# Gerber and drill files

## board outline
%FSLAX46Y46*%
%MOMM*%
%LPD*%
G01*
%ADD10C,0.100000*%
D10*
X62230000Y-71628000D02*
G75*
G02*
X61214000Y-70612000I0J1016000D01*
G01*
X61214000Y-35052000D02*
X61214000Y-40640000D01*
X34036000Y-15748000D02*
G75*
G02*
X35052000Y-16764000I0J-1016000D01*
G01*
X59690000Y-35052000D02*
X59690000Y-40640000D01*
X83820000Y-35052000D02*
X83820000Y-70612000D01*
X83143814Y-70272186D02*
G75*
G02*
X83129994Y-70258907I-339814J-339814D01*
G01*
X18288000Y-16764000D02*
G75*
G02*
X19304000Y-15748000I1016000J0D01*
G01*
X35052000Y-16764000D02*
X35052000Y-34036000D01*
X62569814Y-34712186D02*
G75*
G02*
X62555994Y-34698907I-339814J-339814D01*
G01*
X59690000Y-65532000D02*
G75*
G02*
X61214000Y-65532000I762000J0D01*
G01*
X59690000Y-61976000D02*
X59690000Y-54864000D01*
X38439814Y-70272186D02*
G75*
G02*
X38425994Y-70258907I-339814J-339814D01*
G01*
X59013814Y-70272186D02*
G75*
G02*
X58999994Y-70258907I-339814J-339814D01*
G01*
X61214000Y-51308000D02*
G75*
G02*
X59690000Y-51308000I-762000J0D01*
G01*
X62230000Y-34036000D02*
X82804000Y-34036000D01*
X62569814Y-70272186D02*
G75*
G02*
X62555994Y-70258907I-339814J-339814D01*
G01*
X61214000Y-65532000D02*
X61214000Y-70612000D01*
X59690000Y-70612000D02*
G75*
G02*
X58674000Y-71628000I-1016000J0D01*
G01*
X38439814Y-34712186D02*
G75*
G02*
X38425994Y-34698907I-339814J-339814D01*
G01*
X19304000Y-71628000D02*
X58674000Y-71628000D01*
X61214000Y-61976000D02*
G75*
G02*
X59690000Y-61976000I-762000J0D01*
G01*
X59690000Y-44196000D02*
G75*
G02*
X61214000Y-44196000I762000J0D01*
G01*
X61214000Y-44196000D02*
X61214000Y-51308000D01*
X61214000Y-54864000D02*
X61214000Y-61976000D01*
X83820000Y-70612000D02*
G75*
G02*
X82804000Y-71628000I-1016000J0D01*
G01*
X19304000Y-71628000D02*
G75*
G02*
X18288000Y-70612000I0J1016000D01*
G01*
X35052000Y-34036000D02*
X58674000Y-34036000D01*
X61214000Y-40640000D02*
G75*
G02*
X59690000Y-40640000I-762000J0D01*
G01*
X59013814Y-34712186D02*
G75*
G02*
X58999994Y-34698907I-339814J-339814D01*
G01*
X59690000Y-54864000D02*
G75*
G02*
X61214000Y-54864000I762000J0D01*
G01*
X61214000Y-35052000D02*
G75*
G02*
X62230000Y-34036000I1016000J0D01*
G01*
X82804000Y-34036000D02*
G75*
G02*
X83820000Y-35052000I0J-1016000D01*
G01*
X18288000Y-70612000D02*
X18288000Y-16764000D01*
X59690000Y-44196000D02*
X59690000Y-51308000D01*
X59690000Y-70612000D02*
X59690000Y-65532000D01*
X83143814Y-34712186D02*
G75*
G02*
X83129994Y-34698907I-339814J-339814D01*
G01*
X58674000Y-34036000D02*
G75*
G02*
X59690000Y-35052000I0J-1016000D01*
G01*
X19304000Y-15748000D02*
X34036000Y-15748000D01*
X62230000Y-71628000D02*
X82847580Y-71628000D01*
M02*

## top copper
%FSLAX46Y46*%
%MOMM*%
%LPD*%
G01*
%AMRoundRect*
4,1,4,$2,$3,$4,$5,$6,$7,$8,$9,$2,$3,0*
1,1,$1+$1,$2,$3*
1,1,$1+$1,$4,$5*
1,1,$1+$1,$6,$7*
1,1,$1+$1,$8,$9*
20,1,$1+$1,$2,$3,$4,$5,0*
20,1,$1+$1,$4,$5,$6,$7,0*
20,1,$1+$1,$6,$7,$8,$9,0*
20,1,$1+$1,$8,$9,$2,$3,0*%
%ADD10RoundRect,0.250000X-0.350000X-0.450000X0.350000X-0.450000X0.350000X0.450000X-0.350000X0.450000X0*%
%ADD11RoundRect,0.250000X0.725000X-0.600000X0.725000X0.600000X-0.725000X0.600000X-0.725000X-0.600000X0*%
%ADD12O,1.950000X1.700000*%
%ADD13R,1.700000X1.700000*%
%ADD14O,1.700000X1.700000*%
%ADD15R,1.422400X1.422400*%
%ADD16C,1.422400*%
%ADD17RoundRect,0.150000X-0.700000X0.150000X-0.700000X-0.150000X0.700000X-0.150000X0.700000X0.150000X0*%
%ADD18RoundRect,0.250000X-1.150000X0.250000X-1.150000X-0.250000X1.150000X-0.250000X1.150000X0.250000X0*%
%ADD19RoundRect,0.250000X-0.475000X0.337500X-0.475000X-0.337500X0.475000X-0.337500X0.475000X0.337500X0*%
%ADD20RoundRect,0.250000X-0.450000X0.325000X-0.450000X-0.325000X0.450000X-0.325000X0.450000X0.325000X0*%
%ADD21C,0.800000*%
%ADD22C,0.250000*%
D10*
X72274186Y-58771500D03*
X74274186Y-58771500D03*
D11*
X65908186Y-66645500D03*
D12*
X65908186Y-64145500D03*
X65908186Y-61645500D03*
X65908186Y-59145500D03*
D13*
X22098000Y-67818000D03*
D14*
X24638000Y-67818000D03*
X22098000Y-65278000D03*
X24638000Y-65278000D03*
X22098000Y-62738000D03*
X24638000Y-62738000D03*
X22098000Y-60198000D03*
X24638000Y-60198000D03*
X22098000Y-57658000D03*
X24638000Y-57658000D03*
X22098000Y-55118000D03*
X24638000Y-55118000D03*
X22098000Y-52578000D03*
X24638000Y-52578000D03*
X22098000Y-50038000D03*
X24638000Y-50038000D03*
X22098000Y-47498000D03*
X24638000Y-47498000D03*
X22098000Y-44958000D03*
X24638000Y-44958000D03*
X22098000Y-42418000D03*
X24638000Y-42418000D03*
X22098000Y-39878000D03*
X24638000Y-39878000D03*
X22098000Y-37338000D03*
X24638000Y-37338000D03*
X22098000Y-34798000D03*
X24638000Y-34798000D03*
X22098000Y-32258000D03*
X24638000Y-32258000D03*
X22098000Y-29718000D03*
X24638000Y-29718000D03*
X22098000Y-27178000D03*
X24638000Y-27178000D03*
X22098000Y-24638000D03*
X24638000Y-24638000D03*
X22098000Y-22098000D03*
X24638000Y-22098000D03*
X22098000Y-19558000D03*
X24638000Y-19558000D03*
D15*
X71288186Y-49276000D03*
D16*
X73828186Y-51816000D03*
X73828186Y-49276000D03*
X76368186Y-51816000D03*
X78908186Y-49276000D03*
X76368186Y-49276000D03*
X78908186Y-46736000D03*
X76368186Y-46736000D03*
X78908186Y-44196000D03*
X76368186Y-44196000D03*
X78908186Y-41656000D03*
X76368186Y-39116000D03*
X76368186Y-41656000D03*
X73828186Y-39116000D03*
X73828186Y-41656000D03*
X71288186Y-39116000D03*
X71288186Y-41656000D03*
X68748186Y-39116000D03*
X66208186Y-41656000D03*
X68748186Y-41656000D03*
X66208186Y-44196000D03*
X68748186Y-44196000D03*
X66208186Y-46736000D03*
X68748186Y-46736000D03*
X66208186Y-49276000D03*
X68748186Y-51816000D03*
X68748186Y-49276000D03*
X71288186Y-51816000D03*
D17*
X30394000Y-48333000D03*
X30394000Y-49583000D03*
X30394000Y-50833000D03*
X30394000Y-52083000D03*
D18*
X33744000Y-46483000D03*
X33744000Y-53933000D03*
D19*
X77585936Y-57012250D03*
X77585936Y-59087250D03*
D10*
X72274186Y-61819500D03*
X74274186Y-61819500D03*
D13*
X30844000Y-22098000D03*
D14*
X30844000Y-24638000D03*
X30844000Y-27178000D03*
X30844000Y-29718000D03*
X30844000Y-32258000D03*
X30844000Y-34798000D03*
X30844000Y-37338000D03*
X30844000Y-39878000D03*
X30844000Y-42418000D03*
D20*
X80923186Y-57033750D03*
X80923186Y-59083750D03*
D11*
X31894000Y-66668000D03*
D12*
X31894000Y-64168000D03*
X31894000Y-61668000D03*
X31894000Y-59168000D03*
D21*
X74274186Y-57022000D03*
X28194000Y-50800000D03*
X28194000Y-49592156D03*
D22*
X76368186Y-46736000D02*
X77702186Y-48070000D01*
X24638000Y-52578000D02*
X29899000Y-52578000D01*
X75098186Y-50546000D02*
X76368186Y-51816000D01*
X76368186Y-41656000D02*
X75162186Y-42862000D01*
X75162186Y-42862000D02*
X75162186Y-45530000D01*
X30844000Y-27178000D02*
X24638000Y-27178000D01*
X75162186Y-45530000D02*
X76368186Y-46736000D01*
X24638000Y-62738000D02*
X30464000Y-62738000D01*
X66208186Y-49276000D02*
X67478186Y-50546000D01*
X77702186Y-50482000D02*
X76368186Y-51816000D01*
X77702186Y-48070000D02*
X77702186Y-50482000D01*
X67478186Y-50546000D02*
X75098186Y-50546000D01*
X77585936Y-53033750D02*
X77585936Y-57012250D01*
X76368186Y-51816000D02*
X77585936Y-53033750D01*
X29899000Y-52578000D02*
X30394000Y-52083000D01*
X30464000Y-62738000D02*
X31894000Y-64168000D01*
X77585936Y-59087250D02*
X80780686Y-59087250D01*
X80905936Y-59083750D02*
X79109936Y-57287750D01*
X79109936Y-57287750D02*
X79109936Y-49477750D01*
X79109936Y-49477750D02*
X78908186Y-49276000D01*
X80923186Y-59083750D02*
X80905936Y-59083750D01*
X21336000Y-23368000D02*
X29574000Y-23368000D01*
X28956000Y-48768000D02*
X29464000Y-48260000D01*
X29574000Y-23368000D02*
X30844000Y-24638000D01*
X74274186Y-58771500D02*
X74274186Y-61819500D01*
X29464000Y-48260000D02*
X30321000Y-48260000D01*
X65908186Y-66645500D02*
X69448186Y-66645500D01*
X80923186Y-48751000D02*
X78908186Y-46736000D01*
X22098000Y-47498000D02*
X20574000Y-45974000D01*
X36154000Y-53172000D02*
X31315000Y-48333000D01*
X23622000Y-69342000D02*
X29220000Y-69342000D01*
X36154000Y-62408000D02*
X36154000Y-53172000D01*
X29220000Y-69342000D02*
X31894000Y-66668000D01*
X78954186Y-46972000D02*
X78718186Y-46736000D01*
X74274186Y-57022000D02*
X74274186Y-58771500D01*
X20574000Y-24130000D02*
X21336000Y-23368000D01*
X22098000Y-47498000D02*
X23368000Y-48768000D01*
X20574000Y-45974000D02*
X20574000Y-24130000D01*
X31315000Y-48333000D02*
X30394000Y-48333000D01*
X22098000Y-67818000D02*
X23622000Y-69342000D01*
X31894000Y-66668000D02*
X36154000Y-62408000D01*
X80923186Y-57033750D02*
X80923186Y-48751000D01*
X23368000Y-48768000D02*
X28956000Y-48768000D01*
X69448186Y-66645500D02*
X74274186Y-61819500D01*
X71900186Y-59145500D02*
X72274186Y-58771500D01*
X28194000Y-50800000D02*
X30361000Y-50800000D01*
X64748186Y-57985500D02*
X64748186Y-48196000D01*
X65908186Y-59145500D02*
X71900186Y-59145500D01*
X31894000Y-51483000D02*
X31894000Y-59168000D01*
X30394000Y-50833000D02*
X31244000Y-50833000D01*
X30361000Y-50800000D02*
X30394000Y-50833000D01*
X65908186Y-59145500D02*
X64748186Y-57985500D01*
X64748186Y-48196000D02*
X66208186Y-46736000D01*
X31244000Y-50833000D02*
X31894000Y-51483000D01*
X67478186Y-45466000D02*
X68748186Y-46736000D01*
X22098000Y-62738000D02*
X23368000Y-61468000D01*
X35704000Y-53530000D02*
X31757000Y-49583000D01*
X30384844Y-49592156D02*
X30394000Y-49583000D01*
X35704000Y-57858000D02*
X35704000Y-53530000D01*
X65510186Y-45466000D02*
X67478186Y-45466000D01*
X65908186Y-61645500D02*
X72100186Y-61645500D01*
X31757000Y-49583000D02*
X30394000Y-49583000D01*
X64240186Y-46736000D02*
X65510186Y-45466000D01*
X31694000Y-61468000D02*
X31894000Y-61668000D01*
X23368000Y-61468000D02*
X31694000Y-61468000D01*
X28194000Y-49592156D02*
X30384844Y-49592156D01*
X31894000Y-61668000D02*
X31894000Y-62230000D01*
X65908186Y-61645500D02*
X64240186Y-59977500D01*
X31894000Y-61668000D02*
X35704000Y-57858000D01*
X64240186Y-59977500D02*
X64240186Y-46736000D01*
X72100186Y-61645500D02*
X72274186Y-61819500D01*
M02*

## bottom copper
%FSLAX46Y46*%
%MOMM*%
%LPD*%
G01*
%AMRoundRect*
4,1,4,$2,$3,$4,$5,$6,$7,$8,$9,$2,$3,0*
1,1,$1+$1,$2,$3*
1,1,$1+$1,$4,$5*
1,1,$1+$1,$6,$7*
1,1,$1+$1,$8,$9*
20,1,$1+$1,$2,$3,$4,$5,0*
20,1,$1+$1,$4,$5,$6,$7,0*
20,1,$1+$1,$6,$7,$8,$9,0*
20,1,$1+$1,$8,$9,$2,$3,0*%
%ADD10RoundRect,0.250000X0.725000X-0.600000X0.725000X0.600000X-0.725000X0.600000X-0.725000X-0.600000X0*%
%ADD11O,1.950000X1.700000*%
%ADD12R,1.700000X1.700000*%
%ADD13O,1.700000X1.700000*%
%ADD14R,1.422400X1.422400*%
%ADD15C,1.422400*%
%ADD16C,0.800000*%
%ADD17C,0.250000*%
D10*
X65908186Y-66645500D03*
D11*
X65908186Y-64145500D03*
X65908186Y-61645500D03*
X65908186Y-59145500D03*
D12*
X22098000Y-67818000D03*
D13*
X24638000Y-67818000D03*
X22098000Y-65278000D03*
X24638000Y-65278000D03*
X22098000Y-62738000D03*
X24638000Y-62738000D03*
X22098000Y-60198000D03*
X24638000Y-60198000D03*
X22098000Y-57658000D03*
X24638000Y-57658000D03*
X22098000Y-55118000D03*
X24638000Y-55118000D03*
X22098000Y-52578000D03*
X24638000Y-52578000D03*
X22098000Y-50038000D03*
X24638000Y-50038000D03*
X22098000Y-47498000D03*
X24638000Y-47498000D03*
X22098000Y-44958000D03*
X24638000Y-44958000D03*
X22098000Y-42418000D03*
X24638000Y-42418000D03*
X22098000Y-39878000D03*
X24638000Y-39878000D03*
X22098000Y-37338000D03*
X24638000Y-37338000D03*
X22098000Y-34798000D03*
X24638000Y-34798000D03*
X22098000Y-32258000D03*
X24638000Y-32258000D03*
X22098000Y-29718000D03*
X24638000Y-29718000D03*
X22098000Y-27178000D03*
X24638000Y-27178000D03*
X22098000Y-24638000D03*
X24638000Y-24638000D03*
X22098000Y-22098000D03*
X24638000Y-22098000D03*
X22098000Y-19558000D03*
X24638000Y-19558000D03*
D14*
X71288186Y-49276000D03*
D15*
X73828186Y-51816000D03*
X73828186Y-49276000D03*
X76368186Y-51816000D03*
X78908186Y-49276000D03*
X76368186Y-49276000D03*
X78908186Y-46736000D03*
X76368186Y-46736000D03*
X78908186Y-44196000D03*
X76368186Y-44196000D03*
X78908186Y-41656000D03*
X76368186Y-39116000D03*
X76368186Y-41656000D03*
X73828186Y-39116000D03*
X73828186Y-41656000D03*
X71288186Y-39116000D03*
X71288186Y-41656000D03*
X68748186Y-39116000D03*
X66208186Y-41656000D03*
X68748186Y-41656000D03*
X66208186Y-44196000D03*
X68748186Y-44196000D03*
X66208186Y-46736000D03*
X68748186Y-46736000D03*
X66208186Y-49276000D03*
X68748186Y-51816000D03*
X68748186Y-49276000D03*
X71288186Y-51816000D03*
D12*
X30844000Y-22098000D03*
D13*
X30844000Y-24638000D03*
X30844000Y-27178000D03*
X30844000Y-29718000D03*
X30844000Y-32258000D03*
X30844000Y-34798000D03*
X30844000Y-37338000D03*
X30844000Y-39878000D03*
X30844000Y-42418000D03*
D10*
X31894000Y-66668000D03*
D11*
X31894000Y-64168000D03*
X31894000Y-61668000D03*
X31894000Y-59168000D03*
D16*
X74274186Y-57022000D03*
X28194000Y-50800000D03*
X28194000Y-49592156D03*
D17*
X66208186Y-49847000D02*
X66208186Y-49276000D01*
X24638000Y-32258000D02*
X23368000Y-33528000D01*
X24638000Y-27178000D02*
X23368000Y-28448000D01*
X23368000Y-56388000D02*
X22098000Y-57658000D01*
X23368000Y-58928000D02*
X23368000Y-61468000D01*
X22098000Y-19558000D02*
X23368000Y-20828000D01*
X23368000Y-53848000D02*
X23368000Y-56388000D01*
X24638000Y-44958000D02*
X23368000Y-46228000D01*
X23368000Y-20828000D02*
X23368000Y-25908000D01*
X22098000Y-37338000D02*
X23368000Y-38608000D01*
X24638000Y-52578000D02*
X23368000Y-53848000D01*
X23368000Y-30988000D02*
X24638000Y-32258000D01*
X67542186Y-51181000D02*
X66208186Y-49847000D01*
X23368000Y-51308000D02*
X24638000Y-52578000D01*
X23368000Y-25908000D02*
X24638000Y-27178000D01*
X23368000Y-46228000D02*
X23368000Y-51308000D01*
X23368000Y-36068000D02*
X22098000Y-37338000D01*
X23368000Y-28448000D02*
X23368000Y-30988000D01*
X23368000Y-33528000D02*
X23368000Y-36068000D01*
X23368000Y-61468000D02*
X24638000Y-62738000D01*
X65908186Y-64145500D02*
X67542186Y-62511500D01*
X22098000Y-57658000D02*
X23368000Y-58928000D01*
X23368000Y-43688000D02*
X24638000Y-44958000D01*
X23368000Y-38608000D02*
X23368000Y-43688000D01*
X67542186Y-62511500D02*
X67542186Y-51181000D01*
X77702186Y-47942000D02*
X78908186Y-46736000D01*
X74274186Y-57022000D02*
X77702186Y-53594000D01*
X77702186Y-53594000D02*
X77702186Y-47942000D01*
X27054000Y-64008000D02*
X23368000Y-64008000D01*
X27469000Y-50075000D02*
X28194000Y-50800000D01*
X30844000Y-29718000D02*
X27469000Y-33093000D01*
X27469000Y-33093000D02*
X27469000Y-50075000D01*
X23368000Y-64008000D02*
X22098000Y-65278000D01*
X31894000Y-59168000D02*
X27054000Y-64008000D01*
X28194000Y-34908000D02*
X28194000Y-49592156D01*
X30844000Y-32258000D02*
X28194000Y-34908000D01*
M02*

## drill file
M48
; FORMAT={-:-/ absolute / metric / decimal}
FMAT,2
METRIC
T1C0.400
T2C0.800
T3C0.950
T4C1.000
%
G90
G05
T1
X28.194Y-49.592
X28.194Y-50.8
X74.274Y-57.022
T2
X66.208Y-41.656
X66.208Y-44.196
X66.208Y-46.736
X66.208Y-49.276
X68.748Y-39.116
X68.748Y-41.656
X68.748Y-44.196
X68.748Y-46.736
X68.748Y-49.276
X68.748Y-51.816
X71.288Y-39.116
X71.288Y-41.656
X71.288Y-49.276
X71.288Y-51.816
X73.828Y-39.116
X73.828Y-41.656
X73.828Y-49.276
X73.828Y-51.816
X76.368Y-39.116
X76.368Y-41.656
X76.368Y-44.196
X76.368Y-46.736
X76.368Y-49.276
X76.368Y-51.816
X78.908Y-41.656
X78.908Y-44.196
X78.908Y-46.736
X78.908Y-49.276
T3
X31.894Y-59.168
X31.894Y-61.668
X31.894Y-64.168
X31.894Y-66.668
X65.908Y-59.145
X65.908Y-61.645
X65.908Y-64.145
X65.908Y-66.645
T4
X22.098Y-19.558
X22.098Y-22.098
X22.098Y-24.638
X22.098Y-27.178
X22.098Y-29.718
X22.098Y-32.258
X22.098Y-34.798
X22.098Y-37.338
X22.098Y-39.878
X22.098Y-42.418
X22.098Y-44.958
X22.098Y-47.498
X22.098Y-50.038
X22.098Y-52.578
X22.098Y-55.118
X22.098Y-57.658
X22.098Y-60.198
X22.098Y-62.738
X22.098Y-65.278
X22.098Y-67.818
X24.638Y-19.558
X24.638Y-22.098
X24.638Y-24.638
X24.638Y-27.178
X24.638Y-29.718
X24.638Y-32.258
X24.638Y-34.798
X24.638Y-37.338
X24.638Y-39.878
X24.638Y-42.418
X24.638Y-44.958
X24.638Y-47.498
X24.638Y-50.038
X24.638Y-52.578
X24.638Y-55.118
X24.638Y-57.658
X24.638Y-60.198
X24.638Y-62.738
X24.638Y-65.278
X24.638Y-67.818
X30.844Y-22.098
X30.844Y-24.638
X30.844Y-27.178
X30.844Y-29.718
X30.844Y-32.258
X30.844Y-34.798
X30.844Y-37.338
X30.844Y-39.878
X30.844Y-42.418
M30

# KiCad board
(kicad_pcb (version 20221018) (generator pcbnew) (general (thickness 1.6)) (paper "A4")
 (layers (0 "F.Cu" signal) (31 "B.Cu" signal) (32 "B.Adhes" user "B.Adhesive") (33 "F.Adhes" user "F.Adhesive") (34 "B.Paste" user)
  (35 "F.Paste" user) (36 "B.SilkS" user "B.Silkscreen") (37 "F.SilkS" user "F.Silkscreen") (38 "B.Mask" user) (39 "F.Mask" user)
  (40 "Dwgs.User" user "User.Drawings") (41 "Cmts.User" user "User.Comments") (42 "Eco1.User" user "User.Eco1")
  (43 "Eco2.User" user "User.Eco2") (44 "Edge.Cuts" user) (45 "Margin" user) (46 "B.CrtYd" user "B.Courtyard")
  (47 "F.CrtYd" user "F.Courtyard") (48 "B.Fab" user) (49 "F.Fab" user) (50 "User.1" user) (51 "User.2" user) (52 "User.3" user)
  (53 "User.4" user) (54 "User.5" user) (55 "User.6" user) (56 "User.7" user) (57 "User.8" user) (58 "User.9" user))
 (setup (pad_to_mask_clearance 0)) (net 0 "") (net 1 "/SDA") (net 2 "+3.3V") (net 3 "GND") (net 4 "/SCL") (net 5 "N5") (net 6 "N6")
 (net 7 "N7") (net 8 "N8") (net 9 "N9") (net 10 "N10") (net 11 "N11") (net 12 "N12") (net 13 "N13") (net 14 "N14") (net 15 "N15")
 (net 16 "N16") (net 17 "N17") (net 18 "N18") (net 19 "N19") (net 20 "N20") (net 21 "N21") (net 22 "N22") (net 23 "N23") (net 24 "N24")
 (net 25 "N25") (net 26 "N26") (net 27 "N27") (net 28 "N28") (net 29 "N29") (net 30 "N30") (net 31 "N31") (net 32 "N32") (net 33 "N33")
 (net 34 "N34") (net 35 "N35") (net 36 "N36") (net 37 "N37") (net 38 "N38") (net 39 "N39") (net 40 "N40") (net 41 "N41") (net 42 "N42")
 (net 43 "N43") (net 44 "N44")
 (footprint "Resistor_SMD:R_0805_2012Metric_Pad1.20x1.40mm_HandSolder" (layer "F.Cu") (at 73.274186 58.7715)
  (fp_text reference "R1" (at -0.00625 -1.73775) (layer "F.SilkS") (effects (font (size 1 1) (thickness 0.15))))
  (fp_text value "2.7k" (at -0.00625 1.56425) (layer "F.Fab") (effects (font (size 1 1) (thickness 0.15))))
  (pad "1" smd roundrect (at -1 0) (size 1.2 1.4) (layers "F.Cu" "F.Paste" "F.Mask") (roundrect_rratio 0.208333) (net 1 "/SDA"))
  (pad "2" smd roundrect (at 1 0) (size 1.2 1.4) (layers "F.Cu" "F.Paste" "F.Mask") (roundrect_rratio 0.208333) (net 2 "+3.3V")))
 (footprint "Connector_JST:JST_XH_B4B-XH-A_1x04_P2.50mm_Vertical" (layer "F.Cu") (at 65.908186 66.6455 90)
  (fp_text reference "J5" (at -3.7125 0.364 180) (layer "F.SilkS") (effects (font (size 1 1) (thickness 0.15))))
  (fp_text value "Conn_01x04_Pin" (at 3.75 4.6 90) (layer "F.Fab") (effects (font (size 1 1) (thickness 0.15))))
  (pad "1" thru_hole roundrect (at 0 0 90) (size 1.7 1.95) (drill 0.95) (layers "*.Cu" "*.Mask") (roundrect_rratio 0.147059) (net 2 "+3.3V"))
  (pad "2" thru_hole oval (at 2.5 0 90) (size 1.7 1.95) (drill 0.95) (layers "*.Cu" "*.Mask") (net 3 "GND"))
  (pad "3" thru_hole oval (at 5 0 90) (size 1.7 1.95) (drill 0.95) (layers "*.Cu" "*.Mask") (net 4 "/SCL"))
  (pad "4" thru_hole oval (at 7.5 0 90) (size 1.7 1.95) (drill 0.95) (layers "*.Cu" "*.Mask") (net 1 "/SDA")))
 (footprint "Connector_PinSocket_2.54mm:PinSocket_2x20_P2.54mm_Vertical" (layer "F.Cu") (at 22.098 67.818 180)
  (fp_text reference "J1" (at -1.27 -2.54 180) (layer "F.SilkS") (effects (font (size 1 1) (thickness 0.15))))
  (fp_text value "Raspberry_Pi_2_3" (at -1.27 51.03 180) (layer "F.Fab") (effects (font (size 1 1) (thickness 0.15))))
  (pad "1" thru_hole rect (at 0 0 180) (size 1.7 1.7) (drill 1) (layers "*.Cu" "*.Mask") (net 2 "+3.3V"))
  (pad "2" thru_hole oval (at -2.54 0 180) (size 1.7 1.7) (drill 1) (layers "*.Cu" "*.Mask") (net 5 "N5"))
  (pad "3" thru_hole oval (at 0 2.54 180) (size 1.7 1.7) (drill 1) (layers "*.Cu" "*.Mask") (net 1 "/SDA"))
  (pad "4" thru_hole oval (at -2.54 2.54 180) (size 1.7 1.7) (drill 1) (layers "*.Cu" "*.Mask") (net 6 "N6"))
  (pad "5" thru_hole oval (at 0 5.08 180) (size 1.7 1.7) (drill 1) (layers "*.Cu" "*.Mask") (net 4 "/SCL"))
  (pad "6" thru_hole oval (at -2.54 5.08 180) (size 1.7 1.7) (drill 1) (layers "*.Cu" "*.Mask") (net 3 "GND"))
  (pad "7" thru_hole oval (at 0 7.62 180) (size 1.7 1.7) (drill 1) (layers "*.Cu" "*.Mask") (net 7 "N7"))
  (pad "8" thru_hole oval (at -2.54 7.62 180) (size 1.7 1.7) (drill 1) (layers "*.Cu" "*.Mask") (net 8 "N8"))
  (pad "9" thru_hole oval (at 0 10.16 180) (size 1.7 1.7) (drill 1) (layers "*.Cu" "*.Mask") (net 3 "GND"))
  (pad "10" thru_hole oval (at -2.54 10.16 180) (size 1.7 1.7) (drill 1) (layers "*.Cu" "*.Mask") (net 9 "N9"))
  (pad "11" thru_hole oval (at 0 12.7 180) (size 1.7 1.7) (drill 1) (layers "*.Cu" "*.Mask") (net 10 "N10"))
  (pad "12" thru_hole oval (at -2.54 12.7 180) (size 1.7 1.7) (drill 1) (layers "*.Cu" "*.Mask") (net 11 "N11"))
  (pad "13" thru_hole oval (at 0 15.24 180) (size 1.7 1.7) (drill 1) (layers "*.Cu" "*.Mask") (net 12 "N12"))
  (pad "14" thru_hole oval (at -2.54 15.24 180) (size 1.7 1.7) (drill 1) (layers "*.Cu" "*.Mask") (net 3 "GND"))
  (pad "15" thru_hole oval (at 0 17.78 180) (size 1.7 1.7) (drill 1) (layers "*.Cu" "*.Mask") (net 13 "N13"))
  (pad "16" thru_hole oval (at -2.54 17.78 180) (size 1.7 1.7) (drill 1) (layers "*.Cu" "*.Mask") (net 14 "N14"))
  (pad "17" thru_hole oval (at 0 20.32 180) (size 1.7 1.7) (drill 1) (layers "*.Cu" "*.Mask") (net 2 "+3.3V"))
  (pad "18" thru_hole oval (at -2.54 20.32 180) (size 1.7 1.7) (drill 1) (layers "*.Cu" "*.Mask") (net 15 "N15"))
  (pad "19" thru_hole oval (at 0 22.86 180) (size 1.7 1.7) (drill 1) (layers "*.Cu" "*.Mask") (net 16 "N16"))
  (pad "20" thru_hole oval (at -2.54 22.86 180) (size 1.7 1.7) (drill 1) (layers "*.Cu" "*.Mask") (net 3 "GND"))
  (pad "21" thru_hole oval (at 0 25.4 180) (size 1.7 1.7) (drill 1) (layers "*.Cu" "*.Mask") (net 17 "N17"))
  (pad "22" thru_hole oval (at -2.54 25.4 180) (size 1.7 1.7) (drill 1) (layers "*.Cu" "*.Mask") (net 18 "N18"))
  (pad "23" thru_hole oval (at 0 27.94 180) (size 1.7 1.7) (drill 1) (layers "*.Cu" "*.Mask") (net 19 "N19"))
  (pad "24" thru_hole oval (at -2.54 27.94 180) (size 1.7 1.7) (drill 1) (layers "*.Cu" "*.Mask") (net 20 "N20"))
  (pad "25" thru_hole oval (at 0 30.48 180) (size 1.7 1.7) (drill 1) (layers "*.Cu" "*.Mask") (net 3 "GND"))
  (pad "26" thru_hole oval (at -2.54 30.48 180) (size 1.7 1.7) (drill 1) (layers "*.Cu" "*.Mask") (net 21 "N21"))
  (pad "27" thru_hole oval (at 0 33.02 180) (size 1.7 1.7) (drill 1) (layers "*.Cu" "*.Mask") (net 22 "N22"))
  (pad "28" thru_hole oval (at -2.54 33.02 180) (size 1.7 1.7) (drill 1) (layers "*.Cu" "*.Mask") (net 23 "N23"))
  (pad "29" thru_hole oval (at 0 35.56 180) (size 1.7 1.7) (drill 1) (layers "*.Cu" "*.Mask") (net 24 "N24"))
  (pad "30" thru_hole oval (at -2.54 35.56 180) (size 1.7 1.7) (drill 1) (layers "*.Cu" "*.Mask") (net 3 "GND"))
  (pad "31" thru_hole oval (at 0 38.1 180) (size 1.7 1.7) (drill 1) (layers "*.Cu" "*.Mask") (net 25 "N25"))
  (pad "32" thru_hole oval (at -2.54 38.1 180) (size 1.7 1.7) (drill 1) (layers "*.Cu" "*.Mask") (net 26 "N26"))
  (pad "33" thru_hole oval (at 0 40.64 180) (size 1.7 1.7) (drill 1) (layers "*.Cu" "*.Mask") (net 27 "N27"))
  (pad "34" thru_hole oval (at -2.54 40.64 180) (size 1.7 1.7) (drill 1) (layers "*.Cu" "*.Mask") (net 3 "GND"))
  (pad "35" thru_hole oval (at 0 43.18 180) (size 1.7 1.7) (drill 1) (layers "*.Cu" "*.Mask") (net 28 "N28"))
  (pad "36" thru_hole oval (at -2.54 43.18 180) (size 1.7 1.7) (drill 1) (layers "*.Cu" "*.Mask") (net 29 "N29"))
  (pad "37" thru_hole oval (at 0 45.72 180) (size 1.7 1.7) (drill 1) (layers "*.Cu" "*.Mask") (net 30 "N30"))
  (pad "38" thru_hole oval (at -2.54 45.72 180) (size 1.7 1.7) (drill 1) (layers "*.Cu" "*.Mask") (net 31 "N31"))
  (pad "39" thru_hole oval (at 0 48.26 180) (size 1.7 1.7) (drill 1) (layers "*.Cu" "*.Mask") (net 3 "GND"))
  (pad "40" thru_hole oval (at -2.54 48.26 180) (size 1.7 1.7) (drill 1) (layers "*.Cu" "*.Mask") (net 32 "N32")))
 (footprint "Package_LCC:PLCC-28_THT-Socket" (layer "F.Cu") (at 71.288186 49.276 180)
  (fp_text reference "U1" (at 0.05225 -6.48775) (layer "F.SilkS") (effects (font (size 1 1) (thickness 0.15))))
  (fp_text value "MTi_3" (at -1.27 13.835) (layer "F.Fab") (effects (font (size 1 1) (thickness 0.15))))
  (pad "1" thru_hole rect (at 0 0 180) (size 1.4224 1.4224) (drill 0.8) (layers "*.Cu" "*.Mask"))
  (pad "2" thru_hole circle (at -2.54 -2.54 180) (size 1.4224 1.4224) (drill 0.8) (layers "*.Cu" "*.Mask"))
  (pad "3" thru_hole circle (at -2.54 0 180) (size 1.4224 1.4224) (drill 0.8) (layers "*.Cu" "*.Mask"))
  (pad "4" thru_hole circle (at -5.08 -2.54 180) (size 1.4224 1.4224) (drill 0.8) (layers "*.Cu" "*.Mask") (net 3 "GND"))
  (pad "5" thru_hole circle (at -7.62 0 180) (size 1.4224 1.4224) (drill 0.8) (layers "*.Cu" "*.Mask") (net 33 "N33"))
  (pad "6" thru_hole circle (at -5.08 0 180) (size 1.4224 1.4224) (drill 0.8) (layers "*.Cu" "*.Mask") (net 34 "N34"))
  (pad "7" thru_hole circle (at -7.62 2.54 180) (size 1.4224 1.4224) (drill 0.8) (layers "*.Cu" "*.Mask") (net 2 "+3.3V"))
  (pad "8" thru_hole circle (at -5.08 2.54 180) (size 1.4224 1.4224) (drill 0.8) (layers "*.Cu" "*.Mask") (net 3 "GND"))
  (pad "9" thru_hole circle (at -7.62 5.08 180) (size 1.4224 1.4224) (drill 0.8) (layers "*.Cu" "*.Mask"))
  (pad "10" thru_hole circle (at -5.08 5.08 180) (size 1.4224 1.4224) (drill 0.8) (layers "*.Cu" "*.Mask") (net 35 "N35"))
  (pad "11" thru_hole circle (at -7.62 7.62 180) (size 1.4224 1.4224) (drill 0.8) (layers "*.Cu" "*.Mask") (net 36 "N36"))
  (pad "12" thru_hole circle (at -5.08 10.16 180) (size 1.4224 1.4224) (drill 0.8) (layers "*.Cu" "*.Mask") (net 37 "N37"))
  (pad "13" thru_hole circle (at -5.08 7.62 180) (size 1.4224 1.4224) (drill 0.8) (layers "*.Cu" "*.Mask") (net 3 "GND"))
  (pad "14" thru_hole circle (at -2.54 10.16 180) (size 1.4224 1.4224) (drill 0.8) (layers "*.Cu" "*.Mask") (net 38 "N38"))
  (pad "15" thru_hole circle (at -2.54 7.62 180) (size 1.4224 1.4224) (drill 0.8) (layers "*.Cu" "*.Mask") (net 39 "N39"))
  (pad "16" thru_hole circle (at 0 10.16 180) (size 1.4224 1.4224) (drill 0.8) (layers "*.Cu" "*.Mask"))
  (pad "17" thru_hole circle (at 0 7.62 180) (size 1.4224 1.4224) (drill 0.8) (layers "*.Cu" "*.Mask"))
  (pad "18" thru_hole circle (at 2.54 10.16 180) (size 1.4224 1.4224) (drill 0.8) (layers "*.Cu" "*.Mask"))
  (pad "19" thru_hole circle (at 5.08 7.62 180) (size 1.4224 1.4224) (drill 0.8) (layers "*.Cu" "*.Mask"))
  (pad "20" thru_hole circle (at 2.54 7.62 180) (size 1.4224 1.4224) (drill 0.8) (layers "*.Cu" "*.Mask"))
  (pad "21" thru_hole circle (at 5.08 5.08 180) (size 1.4224 1.4224) (drill 0.8) (layers "*.Cu" "*.Mask"))
  (pad "22" thru_hole circle (at 2.54 5.08 180) (size 1.4224 1.4224) (drill 0.8) (layers "*.Cu" "*.Mask"))
  (pad "23" thru_hole circle (at 5.08 2.54 180) (size 1.4224 1.4224) (drill 0.8) (layers "*.Cu" "*.Mask") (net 1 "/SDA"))
  (pad "24" thru_hole circle (at 2.54 2.54 180) (size 1.4224 1.4224) (drill 0.8) (layers "*.Cu" "*.Mask") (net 4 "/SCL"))
  (pad "25" thru_hole circle (at 5.08 0 180) (size 1.4224 1.4224) (drill 0.8) (layers "*.Cu" "*.Mask") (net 3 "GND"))
  (pad "26" thru_hole circle (at 2.54 -2.54 180) (size 1.4224 1.4224) (drill 0.8) (layers "*.Cu" "*.Mask"))
  (pad "27" thru_hole circle (at 2.54 0 180) (size 1.4224 1.4224) (drill 0.8) (layers "*.Cu" "*.Mask"))
  (pad "28" thru_hole circle (at 0 -2.54 180) (size 1.4224 1.4224) (drill 0.8) (layers "*.Cu" "*.Mask")))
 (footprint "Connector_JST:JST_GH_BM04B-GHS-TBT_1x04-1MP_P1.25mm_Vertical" (layer "F.Cu") (at 32.344 50.208 -90)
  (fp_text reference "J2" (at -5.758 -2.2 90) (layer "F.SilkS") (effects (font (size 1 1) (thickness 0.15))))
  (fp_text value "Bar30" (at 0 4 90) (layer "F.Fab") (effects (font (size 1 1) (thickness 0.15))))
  (pad "1" smd roundrect (at -1.875 1.95 270) (size 0.6 1.7) (layers "F.Cu" "F.Paste" "F.Mask") (roundrect_rratio 0.25) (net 2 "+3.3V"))
  (pad "2" smd roundrect (at -0.625 1.95 270) (size 0.6 1.7) (layers "F.Cu" "F.Paste" "F.Mask") (roundrect_rratio 0.25) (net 4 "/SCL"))
  (pad "3" smd roundrect (at 0.625 1.95 270) (size 0.6 1.7) (layers "F.Cu" "F.Paste" "F.Mask") (roundrect_rratio 0.25) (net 1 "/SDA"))
  (pad "4" smd roundrect (at 1.875 1.95 270) (size 0.6 1.7) (layers "F.Cu" "F.Paste" "F.Mask") (roundrect_rratio 0.25) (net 3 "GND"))
  (pad "MP" smd roundrect (at -3.725 -1.4 270) (size 1 2.8) (layers "F.Cu" "F.Paste" "F.Mask") (roundrect_rratio 0.25))
  (pad "MP" smd roundrect (at 3.725 -1.4 270) (size 1 2.8) (layers "F.Cu" "F.Paste" "F.Mask") (roundrect_rratio 0.25)))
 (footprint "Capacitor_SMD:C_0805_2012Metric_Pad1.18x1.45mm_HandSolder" (layer "F.Cu") (at 77.585936 58.04975 -90)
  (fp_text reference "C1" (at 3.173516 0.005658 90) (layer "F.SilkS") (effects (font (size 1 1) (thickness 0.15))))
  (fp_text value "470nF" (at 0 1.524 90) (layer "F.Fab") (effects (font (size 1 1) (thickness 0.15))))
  (pad "1" smd roundrect (at -1.0375 0 270) (size 1.175 1.45) (layers "F.Cu" "F.Paste" "F.Mask") (roundrect_rratio 0.212766) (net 3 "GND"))
  (pad "2" smd roundrect (at 1.0375 0 270) (size 1.175 1.45) (layers "F.Cu" "F.Paste" "F.Mask") (roundrect_rratio 0.212766) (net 33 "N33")))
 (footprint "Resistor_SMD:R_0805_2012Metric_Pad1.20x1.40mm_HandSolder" (layer "F.Cu") (at 73.274186 61.8195)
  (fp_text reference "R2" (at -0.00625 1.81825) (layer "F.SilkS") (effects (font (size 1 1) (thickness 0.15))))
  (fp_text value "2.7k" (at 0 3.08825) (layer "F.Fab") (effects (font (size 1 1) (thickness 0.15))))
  (pad "1" smd roundrect (at -1 0) (size 1.2 1.4) (layers "F.Cu" "F.Paste" "F.Mask") (roundrect_rratio 0.208333) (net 4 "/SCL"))
  (pad "2" smd roundrect (at 1 0) (size 1.2 1.4) (layers "F.Cu" "F.Paste" "F.Mask") (roundrect_rratio 0.208333) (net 2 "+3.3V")))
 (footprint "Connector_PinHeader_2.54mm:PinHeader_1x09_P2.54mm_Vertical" (layer "F.Cu") (at 30.844 22.098)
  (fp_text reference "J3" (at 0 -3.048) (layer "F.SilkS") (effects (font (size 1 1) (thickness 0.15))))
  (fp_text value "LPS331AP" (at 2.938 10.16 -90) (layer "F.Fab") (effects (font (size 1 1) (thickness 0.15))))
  (pad "1" thru_hole rect (at 0 0) (size 1.7 1.7) (drill 1) (layers "*.Cu" "*.Mask") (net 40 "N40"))
  (pad "2" thru_hole oval (at 0 2.54) (size 1.7 1.7) (drill 1) (layers "*.Cu" "*.Mask") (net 2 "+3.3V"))
  (pad "3" thru_hole oval (at 0 5.08) (size 1.7 1.7) (drill 1) (layers "*.Cu" "*.Mask") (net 3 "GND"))
  (pad "4" thru_hole oval (at 0 7.62) (size 1.7 1.7) (drill 1) (layers "*.Cu" "*.Mask") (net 1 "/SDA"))
  (pad "5" thru_hole oval (at 0 10.16) (size 1.7 1.7) (drill 1) (layers "*.Cu" "*.Mask") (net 4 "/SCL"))
  (pad "6" thru_hole oval (at 0 12.7) (size 1.7 1.7) (drill 1) (layers "*.Cu" "*.Mask") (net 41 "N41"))
  (pad "7" thru_hole oval (at 0 15.24) (size 1.7 1.7) (drill 1) (layers "*.Cu" "*.Mask") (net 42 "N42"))
  (pad "8" thru_hole oval (at 0 17.78) (size 1.7 1.7) (drill 1) (layers "*.Cu" "*.Mask") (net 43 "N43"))
  (pad "9" thru_hole oval (at 0 20.32) (size 1.7 1.7) (drill 1) (layers "*.Cu" "*.Mask") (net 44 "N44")))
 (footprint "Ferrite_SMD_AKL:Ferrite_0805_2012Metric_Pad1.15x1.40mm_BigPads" (layer "F.Cu") (at 80.923186 58.05875 -90)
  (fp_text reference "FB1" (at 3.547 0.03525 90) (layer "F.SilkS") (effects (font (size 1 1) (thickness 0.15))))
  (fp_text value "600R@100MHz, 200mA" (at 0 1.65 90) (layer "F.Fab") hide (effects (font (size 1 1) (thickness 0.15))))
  (pad "1" smd roundrect (at -1.025 0 270) (size 1.15 1.4) (layers "F.Cu" "F.Paste" "F.Mask") (roundrect_rratio 0.217391) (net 2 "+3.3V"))
  (pad "2" smd roundrect (at 1.025 0 270) (size 1.15 1.4) (layers "F.Cu" "F.Paste" "F.Mask") (roundrect_rratio 0.217391) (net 33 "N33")))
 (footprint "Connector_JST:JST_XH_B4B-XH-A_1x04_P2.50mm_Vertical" (layer "F.Cu") (at 31.894 66.668 90)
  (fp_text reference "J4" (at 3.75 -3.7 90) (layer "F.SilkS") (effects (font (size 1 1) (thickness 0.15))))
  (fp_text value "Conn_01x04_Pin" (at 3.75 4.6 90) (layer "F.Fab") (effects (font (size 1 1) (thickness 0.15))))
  (pad "1" thru_hole roundrect (at 0 0 90) (size 1.7 1.95) (drill 0.95) (layers "*.Cu" "*.Mask") (roundrect_rratio 0.147059) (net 2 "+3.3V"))
  (pad "2" thru_hole oval (at 2.5 0 90) (size 1.7 1.95) (drill 0.95) (layers "*.Cu" "*.Mask") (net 3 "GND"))
  (pad "3" thru_hole oval (at 5 0 90) (size 1.7 1.95) (drill 0.95) (layers "*.Cu" "*.Mask") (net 4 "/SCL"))
  (pad "4" thru_hole oval (at 7.5 0 90) (size 1.7 1.95) (drill 0.95) (layers "*.Cu" "*.Mask") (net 1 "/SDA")))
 (gr_arc (start 62.23 71.628) (mid 61.51158 71.33042) (end 61.214 70.612) (stroke (width 0.1) (type default)) (layer "Edge.Cuts"))
 (gr_line (start 61.214 35.052) (end 61.214 40.64) (stroke (width 0.1) (type default)) (layer "Edge.Cuts"))
 (gr_arc (start 34.036 15.748) (mid 34.75442 16.04558) (end 35.052 16.764) (stroke (width 0.1) (type default)) (layer "Edge.Cuts"))
 (gr_line (start 59.69 35.052) (end 59.69 40.64) (stroke (width 0.1) (type default)) (layer "Edge.Cuts"))
 (gr_line (start 83.82 35.052) (end 83.82 70.612) (stroke (width 0.1) (type default)) (layer "Edge.Cuts"))
 (gr_arc (start 83.143814 70.272186) (mid 82.47103 70.958523) (end 83.129994 70.258907) (stroke (width 0.1) (type default))
  (layer "Edge.Cuts"))
 (gr_arc (start 18.288 16.764) (mid 18.58558 16.04558) (end 19.304 15.748) (stroke (width 0.1) (type default)) (layer "Edge.Cuts"))
 (gr_line (start 35.052 16.764) (end 35.052 34.036) (stroke (width 0.1) (type default)) (layer "Edge.Cuts"))
 (gr_arc (start 62.569814 34.712186) (mid 61.89703 35.398523) (end 62.555994 34.698907) (stroke (width 0.1) (type default))
  (layer "Edge.Cuts"))
 (gr_arc (start 59.69 65.532) (mid 60.452 64.77) (end 61.214 65.532) (stroke (width 0.1) (type default)) (layer "Edge.Cuts"))
 (gr_line (start 59.69 61.976) (end 59.69 54.864) (stroke (width 0.1) (type default)) (layer "Edge.Cuts"))
 (gr_arc (start 38.439814 70.272186) (mid 37.76703 70.958523) (end 38.425994 70.258907) (stroke (width 0.1) (type default))
  (layer "Edge.Cuts"))
 (gr_arc (start 59.013814 70.272186) (mid 58.34103 70.958523) (end 58.999994 70.258907) (stroke (width 0.1) (type default))
  (layer "Edge.Cuts"))
 (gr_arc (start 61.214 51.308) (mid 60.452 52.07) (end 59.69 51.308) (stroke (width 0.1) (type default)) (layer "Edge.Cuts"))
 (gr_line (start 62.23 34.036) (end 82.804 34.036) (stroke (width 0.1) (type default)) (layer "Edge.Cuts"))
 (gr_arc (start 62.569814 70.272186) (mid 61.89703 70.958523) (end 62.555994 70.258907) (stroke (width 0.1) (type default))
  (layer "Edge.Cuts"))
 (gr_line (start 61.214 65.532) (end 61.214 70.612) (stroke (width 0.1) (type default)) (layer "Edge.Cuts"))
 (gr_arc (start 59.69 70.612) (mid 59.39242 71.33042) (end 58.674 71.628) (stroke (width 0.1) (type default)) (layer "Edge.Cuts"))
 (gr_arc (start 38.439814 34.712186) (mid 37.76703 35.398523) (end 38.425994 34.698907) (stroke (width 0.1) (type default))
  (layer "Edge.Cuts"))
 (gr_line (start 19.304 71.628) (end 58.674 71.628) (stroke (width 0.1) (type default)) (layer "Edge.Cuts"))
 (gr_arc (start 61.214 61.976) (mid 60.452 62.738) (end 59.69 61.976) (stroke (width 0.1) (type default)) (layer "Edge.Cuts"))
 (gr_arc (start 59.69 44.196) (mid 60.452 43.434) (end 61.214 44.196) (stroke (width 0.1) (type default)) (layer "Edge.Cuts"))
 (gr_line (start 61.214 44.196) (end 61.214 51.308) (stroke (width 0.1) (type default)) (layer "Edge.Cuts"))
 (gr_line (start 61.214 54.864) (end 61.214 61.976) (stroke (width 0.1) (type default)) (layer "Edge.Cuts"))
 (gr_arc (start 83.82 70.612) (mid 83.52242 71.33042) (end 82.804 71.628) (stroke (width 0.1) (type default)) (layer "Edge.Cuts"))
 (gr_arc (start 19.304 71.628) (mid 18.58558 71.33042) (end 18.288 70.612) (stroke (width 0.1) (type default)) (layer "Edge.Cuts"))
 (gr_line (start 35.052 34.036) (end 58.674 34.036) (stroke (width 0.1) (type default)) (layer "Edge.Cuts"))
 (gr_arc (start 61.214 40.64) (mid 60.452 41.402) (end 59.69 40.64) (stroke (width 0.1) (type default)) (layer "Edge.Cuts"))
 (gr_arc (start 59.013814 34.712186) (mid 58.34103 35.398523) (end 58.999994 34.698907) (stroke (width 0.1) (type default))
  (layer "Edge.Cuts"))
 (gr_arc (start 59.69 54.864) (mid 60.452 54.102) (end 61.214 54.864) (stroke (width 0.1) (type default)) (layer "Edge.Cuts"))
 (gr_arc (start 61.214 35.052) (mid 61.51158 34.33358) (end 62.23 34.036) (stroke (width 0.1) (type default)) (layer "Edge.Cuts"))
 (gr_arc (start 82.804 34.036) (mid 83.52242 34.33358) (end 83.82 35.052) (stroke (width 0.1) (type default)) (layer "Edge.Cuts"))
 (gr_line (start 18.288 70.612) (end 18.288 16.764) (stroke (width 0.1) (type default)) (layer "Edge.Cuts"))
 (gr_line (start 59.69 44.196) (end 59.69 51.308) (stroke (width 0.1) (type default)) (layer "Edge.Cuts"))
 (gr_line (start 59.69 70.612) (end 59.69 65.532) (stroke (width 0.1) (type default)) (layer "Edge.Cuts"))
 (gr_arc (start 83.143814 34.712186) (mid 82.47103 35.398523) (end 83.129994 34.698907) (stroke (width 0.1) (type default))
  (layer "Edge.Cuts"))
 (gr_arc (start 58.674 34.036) (mid 59.39242 34.33358) (end 59.69 35.052) (stroke (width 0.1) (type default)) (layer "Edge.Cuts"))
 (gr_line (start 19.304 15.748) (end 34.036 15.748) (stroke (width 0.1) (type default)) (layer "Edge.Cuts"))
 (gr_line (start 62.23 71.628) (end 82.84758 71.628) (stroke (width 0.1) (type default)) (layer "Edge.Cuts"))
 (segment (start 76.368186 46.736) (end 77.702186 48.07) (width 0.25) (layer "F.Cu") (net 3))
 (segment (start 24.638 52.578) (end 29.899 52.578) (width 0.25) (layer "F.Cu") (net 3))
 (segment (start 75.098186 50.546) (end 76.368186 51.816) (width 0.25) (layer "F.Cu") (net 3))
 (segment (start 76.368186 41.656) (end 75.162186 42.862) (width 0.25) (layer "F.Cu") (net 3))
 (segment (start 75.162186 42.862) (end 75.162186 45.53) (width 0.25) (layer "F.Cu") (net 3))
 (segment (start 30.844 27.178) (end 24.638 27.178) (width 0.25) (layer "F.Cu") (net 3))
 (segment (start 75.162186 45.53) (end 76.368186 46.736) (width 0.25) (layer "F.Cu") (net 3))
 (segment (start 24.638 62.738) (end 30.464 62.738) (width 0.25) (layer "F.Cu") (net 3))
 (segment (start 66.208186 49.276) (end 67.478186 50.546) (width 0.25) (layer "F.Cu") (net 3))
 (segment (start 77.702186 50.482) (end 76.368186 51.816) (width 0.25) (layer "F.Cu") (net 3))
 (segment (start 77.702186 48.07) (end 77.702186 50.482) (width 0.25) (layer "F.Cu") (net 3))
 (segment (start 67.478186 50.546) (end 75.098186 50.546) (width 0.25) (layer "F.Cu") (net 3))
 (segment (start 77.585936 53.03375) (end 77.585936 57.01225) (width 0.25) (layer "F.Cu") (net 3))
 (segment (start 76.368186 51.816) (end 77.585936 53.03375) (width 0.25) (layer "F.Cu") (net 3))
 (segment (start 29.899 52.578) (end 30.394 52.083) (width 0.25) (layer "F.Cu") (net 3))
 (segment (start 30.464 62.738) (end 31.894 64.168) (width 0.25) (layer "F.Cu") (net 3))
 (segment (start 66.208186 49.847) (end 66.208186 49.276) (width 0.25) (layer "B.Cu") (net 3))
 (segment (start 24.638 32.258) (end 23.368 33.528) (width 0.25) (layer "B.Cu") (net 3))
 (segment (start 24.638 27.178) (end 23.368 28.448) (width 0.25) (layer "B.Cu") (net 3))
 (segment (start 23.368 56.388) (end 22.098 57.658) (width 0.25) (layer "B.Cu") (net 3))
 (segment (start 23.368 58.928) (end 23.368 61.468) (width 0.25) (layer "B.Cu") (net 3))
 (segment (start 22.098 19.558) (end 23.368 20.828) (width 0.25) (layer "B.Cu") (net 3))
 (segment (start 23.368 53.848) (end 23.368 56.388) (width 0.25) (layer "B.Cu") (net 3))
 (segment (start 24.638 44.958) (end 23.368 46.228) (width 0.25) (layer "B.Cu") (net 3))
 (segment (start 23.368 20.828) (end 23.368 25.908) (width 0.25) (layer "B.Cu") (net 3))
 (segment (start 22.098 37.338) (end 23.368 38.608) (width 0.25) (layer "B.Cu") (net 3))
 (segment (start 24.638 52.578) (end 23.368 53.848) (width 0.25) (layer "B.Cu") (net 3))
 (segment (start 23.368 30.988) (end 24.638 32.258) (width 0.25) (layer "B.Cu") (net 3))
 (segment (start 67.542186 51.181) (end 66.208186 49.847) (width 0.25) (layer "B.Cu") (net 3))
 (segment (start 23.368 51.308) (end 24.638 52.578) (width 0.25) (layer "B.Cu") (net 3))
 (segment (start 23.368 25.908) (end 24.638 27.178) (width 0.25) (layer "B.Cu") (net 3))
 (segment (start 23.368 46.228) (end 23.368 51.308) (width 0.25) (layer "B.Cu") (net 3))
 (segment (start 23.368 36.068) (end 22.098 37.338) (width 0.25) (layer "B.Cu") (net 3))
 (segment (start 23.368 28.448) (end 23.368 30.988) (width 0.25) (layer "B.Cu") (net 3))
 (segment (start 23.368 33.528) (end 23.368 36.068) (width 0.25) (layer "B.Cu") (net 3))
 (segment (start 23.368 61.468) (end 24.638 62.738) (width 0.25) (layer "B.Cu") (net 3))
 (segment (start 65.908186 64.1455) (end 67.542186 62.5115) (width 0.25) (layer "B.Cu") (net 3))
 (segment (start 22.098 57.658) (end 23.368 58.928) (width 0.25) (layer "B.Cu") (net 3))
 (segment (start 23.368 43.688) (end 24.638 44.958) (width 0.25) (layer "B.Cu") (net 3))
 (segment (start 23.368 38.608) (end 23.368 43.688) (width 0.25) (layer "B.Cu") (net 3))
 (segment (start 67.542186 62.5115) (end 67.542186 51.181) (width 0.25) (layer "B.Cu") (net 3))
 (segment (start 77.585936 59.08725) (end 80.780686 59.08725) (width 0.25) (layer "F.Cu") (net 33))
 (segment (start 80.905936 59.08375) (end 79.109936 57.28775) (width 0.25) (layer "F.Cu") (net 33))
 (segment (start 79.109936 57.28775) (end 79.109936 49.47775) (width 0.25) (layer "F.Cu") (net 33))
 (segment (start 79.109936 49.47775) (end 78.908186 49.276) (width 0.25) (layer "F.Cu") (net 33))
 (segment (start 80.923186 59.08375) (end 80.905936 59.08375) (width 0.25) (layer "F.Cu") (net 33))
 (segment (start 21.336 23.368) (end 29.574 23.368) (width 0.25) (layer "F.Cu") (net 2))
 (segment (start 28.956 48.768) (end 29.464 48.26) (width 0.25) (layer "F.Cu") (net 2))
 (segment (start 29.574 23.368) (end 30.844 24.638) (width 0.25) (layer "F.Cu") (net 2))
 (segment (start 74.274186 58.7715) (end 74.274186 61.8195) (width 0.25) (layer "F.Cu") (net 2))
 (segment (start 29.464 48.26) (end 30.321 48.26) (width 0.25) (layer "F.Cu") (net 2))
 (segment (start 65.908186 66.6455) (end 69.448186 66.6455) (width 0.25) (layer "F.Cu") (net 2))
 (segment (start 80.923186 48.751) (end 78.908186 46.736) (width 0.25) (layer "F.Cu") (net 2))
 (segment (start 22.098 47.498) (end 20.574 45.974) (width 0.25) (layer "F.Cu") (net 2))
 (segment (start 36.154 53.172) (end 31.315 48.333) (width 0.25) (layer "F.Cu") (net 2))
 (segment (start 23.622 69.342) (end 29.22 69.342) (width 0.25) (layer "F.Cu") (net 2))
 (segment (start 36.154 62.408) (end 36.154 53.172) (width 0.25) (layer "F.Cu") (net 2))
 (segment (start 29.22 69.342) (end 31.894 66.668) (width 0.25) (layer "F.Cu") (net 2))
 (segment (start 78.954186 46.972) (end 78.718186 46.736) (width 0.25) (layer "F.Cu") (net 2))
 (segment (start 74.274186 57.022) (end 74.274186 58.7715) (width 0.25) (layer "F.Cu") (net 2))
 (segment (start 20.574 24.13) (end 21.336 23.368) (width 0.25) (layer "F.Cu") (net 2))
 (segment (start 22.098 47.498) (end 23.368 48.768) (width 0.25) (layer "F.Cu") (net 2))
 (segment (start 20.574 45.974) (end 20.574 24.13) (width 0.25) (layer "F.Cu") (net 2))
 (segment (start 31.315 48.333) (end 30.394 48.333) (width 0.25) (layer "F.Cu") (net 2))
 (segment (start 22.098 67.818) (end 23.622 69.342) (width 0.25) (layer "F.Cu") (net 2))
 (segment (start 31.894 66.668) (end 36.154 62.408) (width 0.25) (layer "F.Cu") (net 2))
 (segment (start 80.923186 57.03375) (end 80.923186 48.751) (width 0.25) (layer "F.Cu") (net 2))
 (segment (start 23.368 48.768) (end 28.956 48.768) (width 0.25) (layer "F.Cu") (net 2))
 (segment (start 69.448186 66.6455) (end 74.274186 61.8195) (width 0.25) (layer "F.Cu") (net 2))
 (via (at 74.274186 57.022) (size 0.8) (drill 0.4) (layers "F.Cu" "B.Cu") (free) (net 2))
 (segment (start 77.702186 47.942) (end 78.908186 46.736) (width 0.25) (layer "B.Cu") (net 2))
 (segment (start 74.274186 57.022) (end 77.702186 53.594) (width 0.25) (layer "B.Cu") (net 2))
 (segment (start 77.702186 53.594) (end 77.702186 47.942) (width 0.25) (layer "B.Cu") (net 2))
 (segment (start 71.900186 59.1455) (end 72.274186 58.7715) (width 0.25) (layer "F.Cu") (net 1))
 (segment (start 28.194 50.8) (end 30.361 50.8) (width 0.25) (layer "F.Cu") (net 1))
 (segment (start 64.748186 57.9855) (end 64.748186 48.196) (width 0.25) (layer "F.Cu") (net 1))
 (segment (start 65.908186 59.1455) (end 71.900186 59.1455) (width 0.25) (layer "F.Cu") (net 1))
 (segment (start 31.894 51.483) (end 31.894 59.168) (width 0.25) (layer "F.Cu") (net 1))
 (segment (start 30.394 50.833) (end 31.244 50.833) (width 0.25) (layer "F.Cu") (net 1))
 (segment (start 30.361 50.8) (end 30.394 50.833) (width 0.25) (layer "F.Cu") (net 1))
 (segment (start 65.908186 59.1455) (end 64.748186 57.9855) (width 0.25) (layer "F.Cu") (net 1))
 (segment (start 64.748186 48.196) (end 66.208186 46.736) (width 0.25) (layer "F.Cu") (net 1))
 (segment (start 31.244 50.833) (end 31.894 51.483) (width 0.25) (layer "F.Cu") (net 1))
 (via (at 28.194 50.8) (size 0.8) (drill 0.4) (layers "F.Cu" "B.Cu") (free) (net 1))
 (segment (start 27.054 64.008) (end 23.368 64.008) (width 0.25) (layer "B.Cu") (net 1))
 (segment (start 27.469 50.075) (end 28.194 50.8) (width 0.25) (layer "B.Cu") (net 1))
 (segment (start 30.844 29.718) (end 27.469 33.093) (width 0.25) (layer "B.Cu") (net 1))
 (segment (start 27.469 33.093) (end 27.469 50.075) (width 0.25) (layer "B.Cu") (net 1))
 (segment (start 23.368 64.008) (end 22.098 65.278) (width 0.25) (layer "B.Cu") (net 1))
 (segment (start 31.894 59.168) (end 27.054 64.008) (width 0.25) (layer "B.Cu") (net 1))
 (segment (start 67.478186 45.466) (end 68.748186 46.736) (width 0.25) (layer "F.Cu") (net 4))
 (segment (start 22.098 62.738) (end 23.368 61.468) (width 0.25) (layer "F.Cu") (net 4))
 (segment (start 35.704 53.53) (end 31.757 49.583) (width 0.25) (layer "F.Cu") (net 4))
 (segment (start 30.384844 49.592156) (end 30.394 49.583) (width 0.25) (layer "F.Cu") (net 4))
 (segment (start 35.704 57.858) (end 35.704 53.53) (width 0.25) (layer "F.Cu") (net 4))
 (segment (start 65.510186 45.466) (end 67.478186 45.466) (width 0.25) (layer "F.Cu") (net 4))
 (segment (start 65.908186 61.6455) (end 72.100186 61.6455) (width 0.25) (layer "F.Cu") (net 4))
 (segment (start 31.757 49.583) (end 30.394 49.583) (width 0.25) (layer "F.Cu") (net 4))
 (segment (start 64.240186 46.736) (end 65.510186 45.466) (width 0.25) (layer "F.Cu") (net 4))
 (segment (start 31.694 61.468) (end 31.894 61.668) (width 0.25) (layer "F.Cu") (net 4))
 (segment (start 23.368 61.468) (end 31.694 61.468) (width 0.25) (layer "F.Cu") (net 4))
 (segment (start 28.194 49.592156) (end 30.384844 49.592156) (width 0.25) (layer "F.Cu") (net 4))
 (segment (start 31.894 61.668) (end 31.894 62.23) (width 0.25) (layer "F.Cu") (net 4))
 (segment (start 65.908186 61.6455) (end 64.240186 59.9775) (width 0.25) (layer "F.Cu") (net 4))
 (segment (start 31.894 61.668) (end 35.704 57.858) (width 0.25) (layer "F.Cu") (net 4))
 (segment (start 64.240186 59.9775) (end 64.240186 46.736) (width 0.25) (layer "F.Cu") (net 4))
 (segment (start 72.100186 61.6455) (end 72.274186 61.8195) (width 0.25) (layer "F.Cu") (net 4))
 (via (at 28.194 49.592156) (size 0.8) (drill 0.4) (layers "F.Cu" "B.Cu") (free) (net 4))
 (segment (start 28.194 34.908) (end 28.194 49.592156) (width 0.25) (layer "B.Cu") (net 4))
 (segment (start 30.844 32.258) (end 28.194 34.908) (width 0.25) (layer "B.Cu") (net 4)))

